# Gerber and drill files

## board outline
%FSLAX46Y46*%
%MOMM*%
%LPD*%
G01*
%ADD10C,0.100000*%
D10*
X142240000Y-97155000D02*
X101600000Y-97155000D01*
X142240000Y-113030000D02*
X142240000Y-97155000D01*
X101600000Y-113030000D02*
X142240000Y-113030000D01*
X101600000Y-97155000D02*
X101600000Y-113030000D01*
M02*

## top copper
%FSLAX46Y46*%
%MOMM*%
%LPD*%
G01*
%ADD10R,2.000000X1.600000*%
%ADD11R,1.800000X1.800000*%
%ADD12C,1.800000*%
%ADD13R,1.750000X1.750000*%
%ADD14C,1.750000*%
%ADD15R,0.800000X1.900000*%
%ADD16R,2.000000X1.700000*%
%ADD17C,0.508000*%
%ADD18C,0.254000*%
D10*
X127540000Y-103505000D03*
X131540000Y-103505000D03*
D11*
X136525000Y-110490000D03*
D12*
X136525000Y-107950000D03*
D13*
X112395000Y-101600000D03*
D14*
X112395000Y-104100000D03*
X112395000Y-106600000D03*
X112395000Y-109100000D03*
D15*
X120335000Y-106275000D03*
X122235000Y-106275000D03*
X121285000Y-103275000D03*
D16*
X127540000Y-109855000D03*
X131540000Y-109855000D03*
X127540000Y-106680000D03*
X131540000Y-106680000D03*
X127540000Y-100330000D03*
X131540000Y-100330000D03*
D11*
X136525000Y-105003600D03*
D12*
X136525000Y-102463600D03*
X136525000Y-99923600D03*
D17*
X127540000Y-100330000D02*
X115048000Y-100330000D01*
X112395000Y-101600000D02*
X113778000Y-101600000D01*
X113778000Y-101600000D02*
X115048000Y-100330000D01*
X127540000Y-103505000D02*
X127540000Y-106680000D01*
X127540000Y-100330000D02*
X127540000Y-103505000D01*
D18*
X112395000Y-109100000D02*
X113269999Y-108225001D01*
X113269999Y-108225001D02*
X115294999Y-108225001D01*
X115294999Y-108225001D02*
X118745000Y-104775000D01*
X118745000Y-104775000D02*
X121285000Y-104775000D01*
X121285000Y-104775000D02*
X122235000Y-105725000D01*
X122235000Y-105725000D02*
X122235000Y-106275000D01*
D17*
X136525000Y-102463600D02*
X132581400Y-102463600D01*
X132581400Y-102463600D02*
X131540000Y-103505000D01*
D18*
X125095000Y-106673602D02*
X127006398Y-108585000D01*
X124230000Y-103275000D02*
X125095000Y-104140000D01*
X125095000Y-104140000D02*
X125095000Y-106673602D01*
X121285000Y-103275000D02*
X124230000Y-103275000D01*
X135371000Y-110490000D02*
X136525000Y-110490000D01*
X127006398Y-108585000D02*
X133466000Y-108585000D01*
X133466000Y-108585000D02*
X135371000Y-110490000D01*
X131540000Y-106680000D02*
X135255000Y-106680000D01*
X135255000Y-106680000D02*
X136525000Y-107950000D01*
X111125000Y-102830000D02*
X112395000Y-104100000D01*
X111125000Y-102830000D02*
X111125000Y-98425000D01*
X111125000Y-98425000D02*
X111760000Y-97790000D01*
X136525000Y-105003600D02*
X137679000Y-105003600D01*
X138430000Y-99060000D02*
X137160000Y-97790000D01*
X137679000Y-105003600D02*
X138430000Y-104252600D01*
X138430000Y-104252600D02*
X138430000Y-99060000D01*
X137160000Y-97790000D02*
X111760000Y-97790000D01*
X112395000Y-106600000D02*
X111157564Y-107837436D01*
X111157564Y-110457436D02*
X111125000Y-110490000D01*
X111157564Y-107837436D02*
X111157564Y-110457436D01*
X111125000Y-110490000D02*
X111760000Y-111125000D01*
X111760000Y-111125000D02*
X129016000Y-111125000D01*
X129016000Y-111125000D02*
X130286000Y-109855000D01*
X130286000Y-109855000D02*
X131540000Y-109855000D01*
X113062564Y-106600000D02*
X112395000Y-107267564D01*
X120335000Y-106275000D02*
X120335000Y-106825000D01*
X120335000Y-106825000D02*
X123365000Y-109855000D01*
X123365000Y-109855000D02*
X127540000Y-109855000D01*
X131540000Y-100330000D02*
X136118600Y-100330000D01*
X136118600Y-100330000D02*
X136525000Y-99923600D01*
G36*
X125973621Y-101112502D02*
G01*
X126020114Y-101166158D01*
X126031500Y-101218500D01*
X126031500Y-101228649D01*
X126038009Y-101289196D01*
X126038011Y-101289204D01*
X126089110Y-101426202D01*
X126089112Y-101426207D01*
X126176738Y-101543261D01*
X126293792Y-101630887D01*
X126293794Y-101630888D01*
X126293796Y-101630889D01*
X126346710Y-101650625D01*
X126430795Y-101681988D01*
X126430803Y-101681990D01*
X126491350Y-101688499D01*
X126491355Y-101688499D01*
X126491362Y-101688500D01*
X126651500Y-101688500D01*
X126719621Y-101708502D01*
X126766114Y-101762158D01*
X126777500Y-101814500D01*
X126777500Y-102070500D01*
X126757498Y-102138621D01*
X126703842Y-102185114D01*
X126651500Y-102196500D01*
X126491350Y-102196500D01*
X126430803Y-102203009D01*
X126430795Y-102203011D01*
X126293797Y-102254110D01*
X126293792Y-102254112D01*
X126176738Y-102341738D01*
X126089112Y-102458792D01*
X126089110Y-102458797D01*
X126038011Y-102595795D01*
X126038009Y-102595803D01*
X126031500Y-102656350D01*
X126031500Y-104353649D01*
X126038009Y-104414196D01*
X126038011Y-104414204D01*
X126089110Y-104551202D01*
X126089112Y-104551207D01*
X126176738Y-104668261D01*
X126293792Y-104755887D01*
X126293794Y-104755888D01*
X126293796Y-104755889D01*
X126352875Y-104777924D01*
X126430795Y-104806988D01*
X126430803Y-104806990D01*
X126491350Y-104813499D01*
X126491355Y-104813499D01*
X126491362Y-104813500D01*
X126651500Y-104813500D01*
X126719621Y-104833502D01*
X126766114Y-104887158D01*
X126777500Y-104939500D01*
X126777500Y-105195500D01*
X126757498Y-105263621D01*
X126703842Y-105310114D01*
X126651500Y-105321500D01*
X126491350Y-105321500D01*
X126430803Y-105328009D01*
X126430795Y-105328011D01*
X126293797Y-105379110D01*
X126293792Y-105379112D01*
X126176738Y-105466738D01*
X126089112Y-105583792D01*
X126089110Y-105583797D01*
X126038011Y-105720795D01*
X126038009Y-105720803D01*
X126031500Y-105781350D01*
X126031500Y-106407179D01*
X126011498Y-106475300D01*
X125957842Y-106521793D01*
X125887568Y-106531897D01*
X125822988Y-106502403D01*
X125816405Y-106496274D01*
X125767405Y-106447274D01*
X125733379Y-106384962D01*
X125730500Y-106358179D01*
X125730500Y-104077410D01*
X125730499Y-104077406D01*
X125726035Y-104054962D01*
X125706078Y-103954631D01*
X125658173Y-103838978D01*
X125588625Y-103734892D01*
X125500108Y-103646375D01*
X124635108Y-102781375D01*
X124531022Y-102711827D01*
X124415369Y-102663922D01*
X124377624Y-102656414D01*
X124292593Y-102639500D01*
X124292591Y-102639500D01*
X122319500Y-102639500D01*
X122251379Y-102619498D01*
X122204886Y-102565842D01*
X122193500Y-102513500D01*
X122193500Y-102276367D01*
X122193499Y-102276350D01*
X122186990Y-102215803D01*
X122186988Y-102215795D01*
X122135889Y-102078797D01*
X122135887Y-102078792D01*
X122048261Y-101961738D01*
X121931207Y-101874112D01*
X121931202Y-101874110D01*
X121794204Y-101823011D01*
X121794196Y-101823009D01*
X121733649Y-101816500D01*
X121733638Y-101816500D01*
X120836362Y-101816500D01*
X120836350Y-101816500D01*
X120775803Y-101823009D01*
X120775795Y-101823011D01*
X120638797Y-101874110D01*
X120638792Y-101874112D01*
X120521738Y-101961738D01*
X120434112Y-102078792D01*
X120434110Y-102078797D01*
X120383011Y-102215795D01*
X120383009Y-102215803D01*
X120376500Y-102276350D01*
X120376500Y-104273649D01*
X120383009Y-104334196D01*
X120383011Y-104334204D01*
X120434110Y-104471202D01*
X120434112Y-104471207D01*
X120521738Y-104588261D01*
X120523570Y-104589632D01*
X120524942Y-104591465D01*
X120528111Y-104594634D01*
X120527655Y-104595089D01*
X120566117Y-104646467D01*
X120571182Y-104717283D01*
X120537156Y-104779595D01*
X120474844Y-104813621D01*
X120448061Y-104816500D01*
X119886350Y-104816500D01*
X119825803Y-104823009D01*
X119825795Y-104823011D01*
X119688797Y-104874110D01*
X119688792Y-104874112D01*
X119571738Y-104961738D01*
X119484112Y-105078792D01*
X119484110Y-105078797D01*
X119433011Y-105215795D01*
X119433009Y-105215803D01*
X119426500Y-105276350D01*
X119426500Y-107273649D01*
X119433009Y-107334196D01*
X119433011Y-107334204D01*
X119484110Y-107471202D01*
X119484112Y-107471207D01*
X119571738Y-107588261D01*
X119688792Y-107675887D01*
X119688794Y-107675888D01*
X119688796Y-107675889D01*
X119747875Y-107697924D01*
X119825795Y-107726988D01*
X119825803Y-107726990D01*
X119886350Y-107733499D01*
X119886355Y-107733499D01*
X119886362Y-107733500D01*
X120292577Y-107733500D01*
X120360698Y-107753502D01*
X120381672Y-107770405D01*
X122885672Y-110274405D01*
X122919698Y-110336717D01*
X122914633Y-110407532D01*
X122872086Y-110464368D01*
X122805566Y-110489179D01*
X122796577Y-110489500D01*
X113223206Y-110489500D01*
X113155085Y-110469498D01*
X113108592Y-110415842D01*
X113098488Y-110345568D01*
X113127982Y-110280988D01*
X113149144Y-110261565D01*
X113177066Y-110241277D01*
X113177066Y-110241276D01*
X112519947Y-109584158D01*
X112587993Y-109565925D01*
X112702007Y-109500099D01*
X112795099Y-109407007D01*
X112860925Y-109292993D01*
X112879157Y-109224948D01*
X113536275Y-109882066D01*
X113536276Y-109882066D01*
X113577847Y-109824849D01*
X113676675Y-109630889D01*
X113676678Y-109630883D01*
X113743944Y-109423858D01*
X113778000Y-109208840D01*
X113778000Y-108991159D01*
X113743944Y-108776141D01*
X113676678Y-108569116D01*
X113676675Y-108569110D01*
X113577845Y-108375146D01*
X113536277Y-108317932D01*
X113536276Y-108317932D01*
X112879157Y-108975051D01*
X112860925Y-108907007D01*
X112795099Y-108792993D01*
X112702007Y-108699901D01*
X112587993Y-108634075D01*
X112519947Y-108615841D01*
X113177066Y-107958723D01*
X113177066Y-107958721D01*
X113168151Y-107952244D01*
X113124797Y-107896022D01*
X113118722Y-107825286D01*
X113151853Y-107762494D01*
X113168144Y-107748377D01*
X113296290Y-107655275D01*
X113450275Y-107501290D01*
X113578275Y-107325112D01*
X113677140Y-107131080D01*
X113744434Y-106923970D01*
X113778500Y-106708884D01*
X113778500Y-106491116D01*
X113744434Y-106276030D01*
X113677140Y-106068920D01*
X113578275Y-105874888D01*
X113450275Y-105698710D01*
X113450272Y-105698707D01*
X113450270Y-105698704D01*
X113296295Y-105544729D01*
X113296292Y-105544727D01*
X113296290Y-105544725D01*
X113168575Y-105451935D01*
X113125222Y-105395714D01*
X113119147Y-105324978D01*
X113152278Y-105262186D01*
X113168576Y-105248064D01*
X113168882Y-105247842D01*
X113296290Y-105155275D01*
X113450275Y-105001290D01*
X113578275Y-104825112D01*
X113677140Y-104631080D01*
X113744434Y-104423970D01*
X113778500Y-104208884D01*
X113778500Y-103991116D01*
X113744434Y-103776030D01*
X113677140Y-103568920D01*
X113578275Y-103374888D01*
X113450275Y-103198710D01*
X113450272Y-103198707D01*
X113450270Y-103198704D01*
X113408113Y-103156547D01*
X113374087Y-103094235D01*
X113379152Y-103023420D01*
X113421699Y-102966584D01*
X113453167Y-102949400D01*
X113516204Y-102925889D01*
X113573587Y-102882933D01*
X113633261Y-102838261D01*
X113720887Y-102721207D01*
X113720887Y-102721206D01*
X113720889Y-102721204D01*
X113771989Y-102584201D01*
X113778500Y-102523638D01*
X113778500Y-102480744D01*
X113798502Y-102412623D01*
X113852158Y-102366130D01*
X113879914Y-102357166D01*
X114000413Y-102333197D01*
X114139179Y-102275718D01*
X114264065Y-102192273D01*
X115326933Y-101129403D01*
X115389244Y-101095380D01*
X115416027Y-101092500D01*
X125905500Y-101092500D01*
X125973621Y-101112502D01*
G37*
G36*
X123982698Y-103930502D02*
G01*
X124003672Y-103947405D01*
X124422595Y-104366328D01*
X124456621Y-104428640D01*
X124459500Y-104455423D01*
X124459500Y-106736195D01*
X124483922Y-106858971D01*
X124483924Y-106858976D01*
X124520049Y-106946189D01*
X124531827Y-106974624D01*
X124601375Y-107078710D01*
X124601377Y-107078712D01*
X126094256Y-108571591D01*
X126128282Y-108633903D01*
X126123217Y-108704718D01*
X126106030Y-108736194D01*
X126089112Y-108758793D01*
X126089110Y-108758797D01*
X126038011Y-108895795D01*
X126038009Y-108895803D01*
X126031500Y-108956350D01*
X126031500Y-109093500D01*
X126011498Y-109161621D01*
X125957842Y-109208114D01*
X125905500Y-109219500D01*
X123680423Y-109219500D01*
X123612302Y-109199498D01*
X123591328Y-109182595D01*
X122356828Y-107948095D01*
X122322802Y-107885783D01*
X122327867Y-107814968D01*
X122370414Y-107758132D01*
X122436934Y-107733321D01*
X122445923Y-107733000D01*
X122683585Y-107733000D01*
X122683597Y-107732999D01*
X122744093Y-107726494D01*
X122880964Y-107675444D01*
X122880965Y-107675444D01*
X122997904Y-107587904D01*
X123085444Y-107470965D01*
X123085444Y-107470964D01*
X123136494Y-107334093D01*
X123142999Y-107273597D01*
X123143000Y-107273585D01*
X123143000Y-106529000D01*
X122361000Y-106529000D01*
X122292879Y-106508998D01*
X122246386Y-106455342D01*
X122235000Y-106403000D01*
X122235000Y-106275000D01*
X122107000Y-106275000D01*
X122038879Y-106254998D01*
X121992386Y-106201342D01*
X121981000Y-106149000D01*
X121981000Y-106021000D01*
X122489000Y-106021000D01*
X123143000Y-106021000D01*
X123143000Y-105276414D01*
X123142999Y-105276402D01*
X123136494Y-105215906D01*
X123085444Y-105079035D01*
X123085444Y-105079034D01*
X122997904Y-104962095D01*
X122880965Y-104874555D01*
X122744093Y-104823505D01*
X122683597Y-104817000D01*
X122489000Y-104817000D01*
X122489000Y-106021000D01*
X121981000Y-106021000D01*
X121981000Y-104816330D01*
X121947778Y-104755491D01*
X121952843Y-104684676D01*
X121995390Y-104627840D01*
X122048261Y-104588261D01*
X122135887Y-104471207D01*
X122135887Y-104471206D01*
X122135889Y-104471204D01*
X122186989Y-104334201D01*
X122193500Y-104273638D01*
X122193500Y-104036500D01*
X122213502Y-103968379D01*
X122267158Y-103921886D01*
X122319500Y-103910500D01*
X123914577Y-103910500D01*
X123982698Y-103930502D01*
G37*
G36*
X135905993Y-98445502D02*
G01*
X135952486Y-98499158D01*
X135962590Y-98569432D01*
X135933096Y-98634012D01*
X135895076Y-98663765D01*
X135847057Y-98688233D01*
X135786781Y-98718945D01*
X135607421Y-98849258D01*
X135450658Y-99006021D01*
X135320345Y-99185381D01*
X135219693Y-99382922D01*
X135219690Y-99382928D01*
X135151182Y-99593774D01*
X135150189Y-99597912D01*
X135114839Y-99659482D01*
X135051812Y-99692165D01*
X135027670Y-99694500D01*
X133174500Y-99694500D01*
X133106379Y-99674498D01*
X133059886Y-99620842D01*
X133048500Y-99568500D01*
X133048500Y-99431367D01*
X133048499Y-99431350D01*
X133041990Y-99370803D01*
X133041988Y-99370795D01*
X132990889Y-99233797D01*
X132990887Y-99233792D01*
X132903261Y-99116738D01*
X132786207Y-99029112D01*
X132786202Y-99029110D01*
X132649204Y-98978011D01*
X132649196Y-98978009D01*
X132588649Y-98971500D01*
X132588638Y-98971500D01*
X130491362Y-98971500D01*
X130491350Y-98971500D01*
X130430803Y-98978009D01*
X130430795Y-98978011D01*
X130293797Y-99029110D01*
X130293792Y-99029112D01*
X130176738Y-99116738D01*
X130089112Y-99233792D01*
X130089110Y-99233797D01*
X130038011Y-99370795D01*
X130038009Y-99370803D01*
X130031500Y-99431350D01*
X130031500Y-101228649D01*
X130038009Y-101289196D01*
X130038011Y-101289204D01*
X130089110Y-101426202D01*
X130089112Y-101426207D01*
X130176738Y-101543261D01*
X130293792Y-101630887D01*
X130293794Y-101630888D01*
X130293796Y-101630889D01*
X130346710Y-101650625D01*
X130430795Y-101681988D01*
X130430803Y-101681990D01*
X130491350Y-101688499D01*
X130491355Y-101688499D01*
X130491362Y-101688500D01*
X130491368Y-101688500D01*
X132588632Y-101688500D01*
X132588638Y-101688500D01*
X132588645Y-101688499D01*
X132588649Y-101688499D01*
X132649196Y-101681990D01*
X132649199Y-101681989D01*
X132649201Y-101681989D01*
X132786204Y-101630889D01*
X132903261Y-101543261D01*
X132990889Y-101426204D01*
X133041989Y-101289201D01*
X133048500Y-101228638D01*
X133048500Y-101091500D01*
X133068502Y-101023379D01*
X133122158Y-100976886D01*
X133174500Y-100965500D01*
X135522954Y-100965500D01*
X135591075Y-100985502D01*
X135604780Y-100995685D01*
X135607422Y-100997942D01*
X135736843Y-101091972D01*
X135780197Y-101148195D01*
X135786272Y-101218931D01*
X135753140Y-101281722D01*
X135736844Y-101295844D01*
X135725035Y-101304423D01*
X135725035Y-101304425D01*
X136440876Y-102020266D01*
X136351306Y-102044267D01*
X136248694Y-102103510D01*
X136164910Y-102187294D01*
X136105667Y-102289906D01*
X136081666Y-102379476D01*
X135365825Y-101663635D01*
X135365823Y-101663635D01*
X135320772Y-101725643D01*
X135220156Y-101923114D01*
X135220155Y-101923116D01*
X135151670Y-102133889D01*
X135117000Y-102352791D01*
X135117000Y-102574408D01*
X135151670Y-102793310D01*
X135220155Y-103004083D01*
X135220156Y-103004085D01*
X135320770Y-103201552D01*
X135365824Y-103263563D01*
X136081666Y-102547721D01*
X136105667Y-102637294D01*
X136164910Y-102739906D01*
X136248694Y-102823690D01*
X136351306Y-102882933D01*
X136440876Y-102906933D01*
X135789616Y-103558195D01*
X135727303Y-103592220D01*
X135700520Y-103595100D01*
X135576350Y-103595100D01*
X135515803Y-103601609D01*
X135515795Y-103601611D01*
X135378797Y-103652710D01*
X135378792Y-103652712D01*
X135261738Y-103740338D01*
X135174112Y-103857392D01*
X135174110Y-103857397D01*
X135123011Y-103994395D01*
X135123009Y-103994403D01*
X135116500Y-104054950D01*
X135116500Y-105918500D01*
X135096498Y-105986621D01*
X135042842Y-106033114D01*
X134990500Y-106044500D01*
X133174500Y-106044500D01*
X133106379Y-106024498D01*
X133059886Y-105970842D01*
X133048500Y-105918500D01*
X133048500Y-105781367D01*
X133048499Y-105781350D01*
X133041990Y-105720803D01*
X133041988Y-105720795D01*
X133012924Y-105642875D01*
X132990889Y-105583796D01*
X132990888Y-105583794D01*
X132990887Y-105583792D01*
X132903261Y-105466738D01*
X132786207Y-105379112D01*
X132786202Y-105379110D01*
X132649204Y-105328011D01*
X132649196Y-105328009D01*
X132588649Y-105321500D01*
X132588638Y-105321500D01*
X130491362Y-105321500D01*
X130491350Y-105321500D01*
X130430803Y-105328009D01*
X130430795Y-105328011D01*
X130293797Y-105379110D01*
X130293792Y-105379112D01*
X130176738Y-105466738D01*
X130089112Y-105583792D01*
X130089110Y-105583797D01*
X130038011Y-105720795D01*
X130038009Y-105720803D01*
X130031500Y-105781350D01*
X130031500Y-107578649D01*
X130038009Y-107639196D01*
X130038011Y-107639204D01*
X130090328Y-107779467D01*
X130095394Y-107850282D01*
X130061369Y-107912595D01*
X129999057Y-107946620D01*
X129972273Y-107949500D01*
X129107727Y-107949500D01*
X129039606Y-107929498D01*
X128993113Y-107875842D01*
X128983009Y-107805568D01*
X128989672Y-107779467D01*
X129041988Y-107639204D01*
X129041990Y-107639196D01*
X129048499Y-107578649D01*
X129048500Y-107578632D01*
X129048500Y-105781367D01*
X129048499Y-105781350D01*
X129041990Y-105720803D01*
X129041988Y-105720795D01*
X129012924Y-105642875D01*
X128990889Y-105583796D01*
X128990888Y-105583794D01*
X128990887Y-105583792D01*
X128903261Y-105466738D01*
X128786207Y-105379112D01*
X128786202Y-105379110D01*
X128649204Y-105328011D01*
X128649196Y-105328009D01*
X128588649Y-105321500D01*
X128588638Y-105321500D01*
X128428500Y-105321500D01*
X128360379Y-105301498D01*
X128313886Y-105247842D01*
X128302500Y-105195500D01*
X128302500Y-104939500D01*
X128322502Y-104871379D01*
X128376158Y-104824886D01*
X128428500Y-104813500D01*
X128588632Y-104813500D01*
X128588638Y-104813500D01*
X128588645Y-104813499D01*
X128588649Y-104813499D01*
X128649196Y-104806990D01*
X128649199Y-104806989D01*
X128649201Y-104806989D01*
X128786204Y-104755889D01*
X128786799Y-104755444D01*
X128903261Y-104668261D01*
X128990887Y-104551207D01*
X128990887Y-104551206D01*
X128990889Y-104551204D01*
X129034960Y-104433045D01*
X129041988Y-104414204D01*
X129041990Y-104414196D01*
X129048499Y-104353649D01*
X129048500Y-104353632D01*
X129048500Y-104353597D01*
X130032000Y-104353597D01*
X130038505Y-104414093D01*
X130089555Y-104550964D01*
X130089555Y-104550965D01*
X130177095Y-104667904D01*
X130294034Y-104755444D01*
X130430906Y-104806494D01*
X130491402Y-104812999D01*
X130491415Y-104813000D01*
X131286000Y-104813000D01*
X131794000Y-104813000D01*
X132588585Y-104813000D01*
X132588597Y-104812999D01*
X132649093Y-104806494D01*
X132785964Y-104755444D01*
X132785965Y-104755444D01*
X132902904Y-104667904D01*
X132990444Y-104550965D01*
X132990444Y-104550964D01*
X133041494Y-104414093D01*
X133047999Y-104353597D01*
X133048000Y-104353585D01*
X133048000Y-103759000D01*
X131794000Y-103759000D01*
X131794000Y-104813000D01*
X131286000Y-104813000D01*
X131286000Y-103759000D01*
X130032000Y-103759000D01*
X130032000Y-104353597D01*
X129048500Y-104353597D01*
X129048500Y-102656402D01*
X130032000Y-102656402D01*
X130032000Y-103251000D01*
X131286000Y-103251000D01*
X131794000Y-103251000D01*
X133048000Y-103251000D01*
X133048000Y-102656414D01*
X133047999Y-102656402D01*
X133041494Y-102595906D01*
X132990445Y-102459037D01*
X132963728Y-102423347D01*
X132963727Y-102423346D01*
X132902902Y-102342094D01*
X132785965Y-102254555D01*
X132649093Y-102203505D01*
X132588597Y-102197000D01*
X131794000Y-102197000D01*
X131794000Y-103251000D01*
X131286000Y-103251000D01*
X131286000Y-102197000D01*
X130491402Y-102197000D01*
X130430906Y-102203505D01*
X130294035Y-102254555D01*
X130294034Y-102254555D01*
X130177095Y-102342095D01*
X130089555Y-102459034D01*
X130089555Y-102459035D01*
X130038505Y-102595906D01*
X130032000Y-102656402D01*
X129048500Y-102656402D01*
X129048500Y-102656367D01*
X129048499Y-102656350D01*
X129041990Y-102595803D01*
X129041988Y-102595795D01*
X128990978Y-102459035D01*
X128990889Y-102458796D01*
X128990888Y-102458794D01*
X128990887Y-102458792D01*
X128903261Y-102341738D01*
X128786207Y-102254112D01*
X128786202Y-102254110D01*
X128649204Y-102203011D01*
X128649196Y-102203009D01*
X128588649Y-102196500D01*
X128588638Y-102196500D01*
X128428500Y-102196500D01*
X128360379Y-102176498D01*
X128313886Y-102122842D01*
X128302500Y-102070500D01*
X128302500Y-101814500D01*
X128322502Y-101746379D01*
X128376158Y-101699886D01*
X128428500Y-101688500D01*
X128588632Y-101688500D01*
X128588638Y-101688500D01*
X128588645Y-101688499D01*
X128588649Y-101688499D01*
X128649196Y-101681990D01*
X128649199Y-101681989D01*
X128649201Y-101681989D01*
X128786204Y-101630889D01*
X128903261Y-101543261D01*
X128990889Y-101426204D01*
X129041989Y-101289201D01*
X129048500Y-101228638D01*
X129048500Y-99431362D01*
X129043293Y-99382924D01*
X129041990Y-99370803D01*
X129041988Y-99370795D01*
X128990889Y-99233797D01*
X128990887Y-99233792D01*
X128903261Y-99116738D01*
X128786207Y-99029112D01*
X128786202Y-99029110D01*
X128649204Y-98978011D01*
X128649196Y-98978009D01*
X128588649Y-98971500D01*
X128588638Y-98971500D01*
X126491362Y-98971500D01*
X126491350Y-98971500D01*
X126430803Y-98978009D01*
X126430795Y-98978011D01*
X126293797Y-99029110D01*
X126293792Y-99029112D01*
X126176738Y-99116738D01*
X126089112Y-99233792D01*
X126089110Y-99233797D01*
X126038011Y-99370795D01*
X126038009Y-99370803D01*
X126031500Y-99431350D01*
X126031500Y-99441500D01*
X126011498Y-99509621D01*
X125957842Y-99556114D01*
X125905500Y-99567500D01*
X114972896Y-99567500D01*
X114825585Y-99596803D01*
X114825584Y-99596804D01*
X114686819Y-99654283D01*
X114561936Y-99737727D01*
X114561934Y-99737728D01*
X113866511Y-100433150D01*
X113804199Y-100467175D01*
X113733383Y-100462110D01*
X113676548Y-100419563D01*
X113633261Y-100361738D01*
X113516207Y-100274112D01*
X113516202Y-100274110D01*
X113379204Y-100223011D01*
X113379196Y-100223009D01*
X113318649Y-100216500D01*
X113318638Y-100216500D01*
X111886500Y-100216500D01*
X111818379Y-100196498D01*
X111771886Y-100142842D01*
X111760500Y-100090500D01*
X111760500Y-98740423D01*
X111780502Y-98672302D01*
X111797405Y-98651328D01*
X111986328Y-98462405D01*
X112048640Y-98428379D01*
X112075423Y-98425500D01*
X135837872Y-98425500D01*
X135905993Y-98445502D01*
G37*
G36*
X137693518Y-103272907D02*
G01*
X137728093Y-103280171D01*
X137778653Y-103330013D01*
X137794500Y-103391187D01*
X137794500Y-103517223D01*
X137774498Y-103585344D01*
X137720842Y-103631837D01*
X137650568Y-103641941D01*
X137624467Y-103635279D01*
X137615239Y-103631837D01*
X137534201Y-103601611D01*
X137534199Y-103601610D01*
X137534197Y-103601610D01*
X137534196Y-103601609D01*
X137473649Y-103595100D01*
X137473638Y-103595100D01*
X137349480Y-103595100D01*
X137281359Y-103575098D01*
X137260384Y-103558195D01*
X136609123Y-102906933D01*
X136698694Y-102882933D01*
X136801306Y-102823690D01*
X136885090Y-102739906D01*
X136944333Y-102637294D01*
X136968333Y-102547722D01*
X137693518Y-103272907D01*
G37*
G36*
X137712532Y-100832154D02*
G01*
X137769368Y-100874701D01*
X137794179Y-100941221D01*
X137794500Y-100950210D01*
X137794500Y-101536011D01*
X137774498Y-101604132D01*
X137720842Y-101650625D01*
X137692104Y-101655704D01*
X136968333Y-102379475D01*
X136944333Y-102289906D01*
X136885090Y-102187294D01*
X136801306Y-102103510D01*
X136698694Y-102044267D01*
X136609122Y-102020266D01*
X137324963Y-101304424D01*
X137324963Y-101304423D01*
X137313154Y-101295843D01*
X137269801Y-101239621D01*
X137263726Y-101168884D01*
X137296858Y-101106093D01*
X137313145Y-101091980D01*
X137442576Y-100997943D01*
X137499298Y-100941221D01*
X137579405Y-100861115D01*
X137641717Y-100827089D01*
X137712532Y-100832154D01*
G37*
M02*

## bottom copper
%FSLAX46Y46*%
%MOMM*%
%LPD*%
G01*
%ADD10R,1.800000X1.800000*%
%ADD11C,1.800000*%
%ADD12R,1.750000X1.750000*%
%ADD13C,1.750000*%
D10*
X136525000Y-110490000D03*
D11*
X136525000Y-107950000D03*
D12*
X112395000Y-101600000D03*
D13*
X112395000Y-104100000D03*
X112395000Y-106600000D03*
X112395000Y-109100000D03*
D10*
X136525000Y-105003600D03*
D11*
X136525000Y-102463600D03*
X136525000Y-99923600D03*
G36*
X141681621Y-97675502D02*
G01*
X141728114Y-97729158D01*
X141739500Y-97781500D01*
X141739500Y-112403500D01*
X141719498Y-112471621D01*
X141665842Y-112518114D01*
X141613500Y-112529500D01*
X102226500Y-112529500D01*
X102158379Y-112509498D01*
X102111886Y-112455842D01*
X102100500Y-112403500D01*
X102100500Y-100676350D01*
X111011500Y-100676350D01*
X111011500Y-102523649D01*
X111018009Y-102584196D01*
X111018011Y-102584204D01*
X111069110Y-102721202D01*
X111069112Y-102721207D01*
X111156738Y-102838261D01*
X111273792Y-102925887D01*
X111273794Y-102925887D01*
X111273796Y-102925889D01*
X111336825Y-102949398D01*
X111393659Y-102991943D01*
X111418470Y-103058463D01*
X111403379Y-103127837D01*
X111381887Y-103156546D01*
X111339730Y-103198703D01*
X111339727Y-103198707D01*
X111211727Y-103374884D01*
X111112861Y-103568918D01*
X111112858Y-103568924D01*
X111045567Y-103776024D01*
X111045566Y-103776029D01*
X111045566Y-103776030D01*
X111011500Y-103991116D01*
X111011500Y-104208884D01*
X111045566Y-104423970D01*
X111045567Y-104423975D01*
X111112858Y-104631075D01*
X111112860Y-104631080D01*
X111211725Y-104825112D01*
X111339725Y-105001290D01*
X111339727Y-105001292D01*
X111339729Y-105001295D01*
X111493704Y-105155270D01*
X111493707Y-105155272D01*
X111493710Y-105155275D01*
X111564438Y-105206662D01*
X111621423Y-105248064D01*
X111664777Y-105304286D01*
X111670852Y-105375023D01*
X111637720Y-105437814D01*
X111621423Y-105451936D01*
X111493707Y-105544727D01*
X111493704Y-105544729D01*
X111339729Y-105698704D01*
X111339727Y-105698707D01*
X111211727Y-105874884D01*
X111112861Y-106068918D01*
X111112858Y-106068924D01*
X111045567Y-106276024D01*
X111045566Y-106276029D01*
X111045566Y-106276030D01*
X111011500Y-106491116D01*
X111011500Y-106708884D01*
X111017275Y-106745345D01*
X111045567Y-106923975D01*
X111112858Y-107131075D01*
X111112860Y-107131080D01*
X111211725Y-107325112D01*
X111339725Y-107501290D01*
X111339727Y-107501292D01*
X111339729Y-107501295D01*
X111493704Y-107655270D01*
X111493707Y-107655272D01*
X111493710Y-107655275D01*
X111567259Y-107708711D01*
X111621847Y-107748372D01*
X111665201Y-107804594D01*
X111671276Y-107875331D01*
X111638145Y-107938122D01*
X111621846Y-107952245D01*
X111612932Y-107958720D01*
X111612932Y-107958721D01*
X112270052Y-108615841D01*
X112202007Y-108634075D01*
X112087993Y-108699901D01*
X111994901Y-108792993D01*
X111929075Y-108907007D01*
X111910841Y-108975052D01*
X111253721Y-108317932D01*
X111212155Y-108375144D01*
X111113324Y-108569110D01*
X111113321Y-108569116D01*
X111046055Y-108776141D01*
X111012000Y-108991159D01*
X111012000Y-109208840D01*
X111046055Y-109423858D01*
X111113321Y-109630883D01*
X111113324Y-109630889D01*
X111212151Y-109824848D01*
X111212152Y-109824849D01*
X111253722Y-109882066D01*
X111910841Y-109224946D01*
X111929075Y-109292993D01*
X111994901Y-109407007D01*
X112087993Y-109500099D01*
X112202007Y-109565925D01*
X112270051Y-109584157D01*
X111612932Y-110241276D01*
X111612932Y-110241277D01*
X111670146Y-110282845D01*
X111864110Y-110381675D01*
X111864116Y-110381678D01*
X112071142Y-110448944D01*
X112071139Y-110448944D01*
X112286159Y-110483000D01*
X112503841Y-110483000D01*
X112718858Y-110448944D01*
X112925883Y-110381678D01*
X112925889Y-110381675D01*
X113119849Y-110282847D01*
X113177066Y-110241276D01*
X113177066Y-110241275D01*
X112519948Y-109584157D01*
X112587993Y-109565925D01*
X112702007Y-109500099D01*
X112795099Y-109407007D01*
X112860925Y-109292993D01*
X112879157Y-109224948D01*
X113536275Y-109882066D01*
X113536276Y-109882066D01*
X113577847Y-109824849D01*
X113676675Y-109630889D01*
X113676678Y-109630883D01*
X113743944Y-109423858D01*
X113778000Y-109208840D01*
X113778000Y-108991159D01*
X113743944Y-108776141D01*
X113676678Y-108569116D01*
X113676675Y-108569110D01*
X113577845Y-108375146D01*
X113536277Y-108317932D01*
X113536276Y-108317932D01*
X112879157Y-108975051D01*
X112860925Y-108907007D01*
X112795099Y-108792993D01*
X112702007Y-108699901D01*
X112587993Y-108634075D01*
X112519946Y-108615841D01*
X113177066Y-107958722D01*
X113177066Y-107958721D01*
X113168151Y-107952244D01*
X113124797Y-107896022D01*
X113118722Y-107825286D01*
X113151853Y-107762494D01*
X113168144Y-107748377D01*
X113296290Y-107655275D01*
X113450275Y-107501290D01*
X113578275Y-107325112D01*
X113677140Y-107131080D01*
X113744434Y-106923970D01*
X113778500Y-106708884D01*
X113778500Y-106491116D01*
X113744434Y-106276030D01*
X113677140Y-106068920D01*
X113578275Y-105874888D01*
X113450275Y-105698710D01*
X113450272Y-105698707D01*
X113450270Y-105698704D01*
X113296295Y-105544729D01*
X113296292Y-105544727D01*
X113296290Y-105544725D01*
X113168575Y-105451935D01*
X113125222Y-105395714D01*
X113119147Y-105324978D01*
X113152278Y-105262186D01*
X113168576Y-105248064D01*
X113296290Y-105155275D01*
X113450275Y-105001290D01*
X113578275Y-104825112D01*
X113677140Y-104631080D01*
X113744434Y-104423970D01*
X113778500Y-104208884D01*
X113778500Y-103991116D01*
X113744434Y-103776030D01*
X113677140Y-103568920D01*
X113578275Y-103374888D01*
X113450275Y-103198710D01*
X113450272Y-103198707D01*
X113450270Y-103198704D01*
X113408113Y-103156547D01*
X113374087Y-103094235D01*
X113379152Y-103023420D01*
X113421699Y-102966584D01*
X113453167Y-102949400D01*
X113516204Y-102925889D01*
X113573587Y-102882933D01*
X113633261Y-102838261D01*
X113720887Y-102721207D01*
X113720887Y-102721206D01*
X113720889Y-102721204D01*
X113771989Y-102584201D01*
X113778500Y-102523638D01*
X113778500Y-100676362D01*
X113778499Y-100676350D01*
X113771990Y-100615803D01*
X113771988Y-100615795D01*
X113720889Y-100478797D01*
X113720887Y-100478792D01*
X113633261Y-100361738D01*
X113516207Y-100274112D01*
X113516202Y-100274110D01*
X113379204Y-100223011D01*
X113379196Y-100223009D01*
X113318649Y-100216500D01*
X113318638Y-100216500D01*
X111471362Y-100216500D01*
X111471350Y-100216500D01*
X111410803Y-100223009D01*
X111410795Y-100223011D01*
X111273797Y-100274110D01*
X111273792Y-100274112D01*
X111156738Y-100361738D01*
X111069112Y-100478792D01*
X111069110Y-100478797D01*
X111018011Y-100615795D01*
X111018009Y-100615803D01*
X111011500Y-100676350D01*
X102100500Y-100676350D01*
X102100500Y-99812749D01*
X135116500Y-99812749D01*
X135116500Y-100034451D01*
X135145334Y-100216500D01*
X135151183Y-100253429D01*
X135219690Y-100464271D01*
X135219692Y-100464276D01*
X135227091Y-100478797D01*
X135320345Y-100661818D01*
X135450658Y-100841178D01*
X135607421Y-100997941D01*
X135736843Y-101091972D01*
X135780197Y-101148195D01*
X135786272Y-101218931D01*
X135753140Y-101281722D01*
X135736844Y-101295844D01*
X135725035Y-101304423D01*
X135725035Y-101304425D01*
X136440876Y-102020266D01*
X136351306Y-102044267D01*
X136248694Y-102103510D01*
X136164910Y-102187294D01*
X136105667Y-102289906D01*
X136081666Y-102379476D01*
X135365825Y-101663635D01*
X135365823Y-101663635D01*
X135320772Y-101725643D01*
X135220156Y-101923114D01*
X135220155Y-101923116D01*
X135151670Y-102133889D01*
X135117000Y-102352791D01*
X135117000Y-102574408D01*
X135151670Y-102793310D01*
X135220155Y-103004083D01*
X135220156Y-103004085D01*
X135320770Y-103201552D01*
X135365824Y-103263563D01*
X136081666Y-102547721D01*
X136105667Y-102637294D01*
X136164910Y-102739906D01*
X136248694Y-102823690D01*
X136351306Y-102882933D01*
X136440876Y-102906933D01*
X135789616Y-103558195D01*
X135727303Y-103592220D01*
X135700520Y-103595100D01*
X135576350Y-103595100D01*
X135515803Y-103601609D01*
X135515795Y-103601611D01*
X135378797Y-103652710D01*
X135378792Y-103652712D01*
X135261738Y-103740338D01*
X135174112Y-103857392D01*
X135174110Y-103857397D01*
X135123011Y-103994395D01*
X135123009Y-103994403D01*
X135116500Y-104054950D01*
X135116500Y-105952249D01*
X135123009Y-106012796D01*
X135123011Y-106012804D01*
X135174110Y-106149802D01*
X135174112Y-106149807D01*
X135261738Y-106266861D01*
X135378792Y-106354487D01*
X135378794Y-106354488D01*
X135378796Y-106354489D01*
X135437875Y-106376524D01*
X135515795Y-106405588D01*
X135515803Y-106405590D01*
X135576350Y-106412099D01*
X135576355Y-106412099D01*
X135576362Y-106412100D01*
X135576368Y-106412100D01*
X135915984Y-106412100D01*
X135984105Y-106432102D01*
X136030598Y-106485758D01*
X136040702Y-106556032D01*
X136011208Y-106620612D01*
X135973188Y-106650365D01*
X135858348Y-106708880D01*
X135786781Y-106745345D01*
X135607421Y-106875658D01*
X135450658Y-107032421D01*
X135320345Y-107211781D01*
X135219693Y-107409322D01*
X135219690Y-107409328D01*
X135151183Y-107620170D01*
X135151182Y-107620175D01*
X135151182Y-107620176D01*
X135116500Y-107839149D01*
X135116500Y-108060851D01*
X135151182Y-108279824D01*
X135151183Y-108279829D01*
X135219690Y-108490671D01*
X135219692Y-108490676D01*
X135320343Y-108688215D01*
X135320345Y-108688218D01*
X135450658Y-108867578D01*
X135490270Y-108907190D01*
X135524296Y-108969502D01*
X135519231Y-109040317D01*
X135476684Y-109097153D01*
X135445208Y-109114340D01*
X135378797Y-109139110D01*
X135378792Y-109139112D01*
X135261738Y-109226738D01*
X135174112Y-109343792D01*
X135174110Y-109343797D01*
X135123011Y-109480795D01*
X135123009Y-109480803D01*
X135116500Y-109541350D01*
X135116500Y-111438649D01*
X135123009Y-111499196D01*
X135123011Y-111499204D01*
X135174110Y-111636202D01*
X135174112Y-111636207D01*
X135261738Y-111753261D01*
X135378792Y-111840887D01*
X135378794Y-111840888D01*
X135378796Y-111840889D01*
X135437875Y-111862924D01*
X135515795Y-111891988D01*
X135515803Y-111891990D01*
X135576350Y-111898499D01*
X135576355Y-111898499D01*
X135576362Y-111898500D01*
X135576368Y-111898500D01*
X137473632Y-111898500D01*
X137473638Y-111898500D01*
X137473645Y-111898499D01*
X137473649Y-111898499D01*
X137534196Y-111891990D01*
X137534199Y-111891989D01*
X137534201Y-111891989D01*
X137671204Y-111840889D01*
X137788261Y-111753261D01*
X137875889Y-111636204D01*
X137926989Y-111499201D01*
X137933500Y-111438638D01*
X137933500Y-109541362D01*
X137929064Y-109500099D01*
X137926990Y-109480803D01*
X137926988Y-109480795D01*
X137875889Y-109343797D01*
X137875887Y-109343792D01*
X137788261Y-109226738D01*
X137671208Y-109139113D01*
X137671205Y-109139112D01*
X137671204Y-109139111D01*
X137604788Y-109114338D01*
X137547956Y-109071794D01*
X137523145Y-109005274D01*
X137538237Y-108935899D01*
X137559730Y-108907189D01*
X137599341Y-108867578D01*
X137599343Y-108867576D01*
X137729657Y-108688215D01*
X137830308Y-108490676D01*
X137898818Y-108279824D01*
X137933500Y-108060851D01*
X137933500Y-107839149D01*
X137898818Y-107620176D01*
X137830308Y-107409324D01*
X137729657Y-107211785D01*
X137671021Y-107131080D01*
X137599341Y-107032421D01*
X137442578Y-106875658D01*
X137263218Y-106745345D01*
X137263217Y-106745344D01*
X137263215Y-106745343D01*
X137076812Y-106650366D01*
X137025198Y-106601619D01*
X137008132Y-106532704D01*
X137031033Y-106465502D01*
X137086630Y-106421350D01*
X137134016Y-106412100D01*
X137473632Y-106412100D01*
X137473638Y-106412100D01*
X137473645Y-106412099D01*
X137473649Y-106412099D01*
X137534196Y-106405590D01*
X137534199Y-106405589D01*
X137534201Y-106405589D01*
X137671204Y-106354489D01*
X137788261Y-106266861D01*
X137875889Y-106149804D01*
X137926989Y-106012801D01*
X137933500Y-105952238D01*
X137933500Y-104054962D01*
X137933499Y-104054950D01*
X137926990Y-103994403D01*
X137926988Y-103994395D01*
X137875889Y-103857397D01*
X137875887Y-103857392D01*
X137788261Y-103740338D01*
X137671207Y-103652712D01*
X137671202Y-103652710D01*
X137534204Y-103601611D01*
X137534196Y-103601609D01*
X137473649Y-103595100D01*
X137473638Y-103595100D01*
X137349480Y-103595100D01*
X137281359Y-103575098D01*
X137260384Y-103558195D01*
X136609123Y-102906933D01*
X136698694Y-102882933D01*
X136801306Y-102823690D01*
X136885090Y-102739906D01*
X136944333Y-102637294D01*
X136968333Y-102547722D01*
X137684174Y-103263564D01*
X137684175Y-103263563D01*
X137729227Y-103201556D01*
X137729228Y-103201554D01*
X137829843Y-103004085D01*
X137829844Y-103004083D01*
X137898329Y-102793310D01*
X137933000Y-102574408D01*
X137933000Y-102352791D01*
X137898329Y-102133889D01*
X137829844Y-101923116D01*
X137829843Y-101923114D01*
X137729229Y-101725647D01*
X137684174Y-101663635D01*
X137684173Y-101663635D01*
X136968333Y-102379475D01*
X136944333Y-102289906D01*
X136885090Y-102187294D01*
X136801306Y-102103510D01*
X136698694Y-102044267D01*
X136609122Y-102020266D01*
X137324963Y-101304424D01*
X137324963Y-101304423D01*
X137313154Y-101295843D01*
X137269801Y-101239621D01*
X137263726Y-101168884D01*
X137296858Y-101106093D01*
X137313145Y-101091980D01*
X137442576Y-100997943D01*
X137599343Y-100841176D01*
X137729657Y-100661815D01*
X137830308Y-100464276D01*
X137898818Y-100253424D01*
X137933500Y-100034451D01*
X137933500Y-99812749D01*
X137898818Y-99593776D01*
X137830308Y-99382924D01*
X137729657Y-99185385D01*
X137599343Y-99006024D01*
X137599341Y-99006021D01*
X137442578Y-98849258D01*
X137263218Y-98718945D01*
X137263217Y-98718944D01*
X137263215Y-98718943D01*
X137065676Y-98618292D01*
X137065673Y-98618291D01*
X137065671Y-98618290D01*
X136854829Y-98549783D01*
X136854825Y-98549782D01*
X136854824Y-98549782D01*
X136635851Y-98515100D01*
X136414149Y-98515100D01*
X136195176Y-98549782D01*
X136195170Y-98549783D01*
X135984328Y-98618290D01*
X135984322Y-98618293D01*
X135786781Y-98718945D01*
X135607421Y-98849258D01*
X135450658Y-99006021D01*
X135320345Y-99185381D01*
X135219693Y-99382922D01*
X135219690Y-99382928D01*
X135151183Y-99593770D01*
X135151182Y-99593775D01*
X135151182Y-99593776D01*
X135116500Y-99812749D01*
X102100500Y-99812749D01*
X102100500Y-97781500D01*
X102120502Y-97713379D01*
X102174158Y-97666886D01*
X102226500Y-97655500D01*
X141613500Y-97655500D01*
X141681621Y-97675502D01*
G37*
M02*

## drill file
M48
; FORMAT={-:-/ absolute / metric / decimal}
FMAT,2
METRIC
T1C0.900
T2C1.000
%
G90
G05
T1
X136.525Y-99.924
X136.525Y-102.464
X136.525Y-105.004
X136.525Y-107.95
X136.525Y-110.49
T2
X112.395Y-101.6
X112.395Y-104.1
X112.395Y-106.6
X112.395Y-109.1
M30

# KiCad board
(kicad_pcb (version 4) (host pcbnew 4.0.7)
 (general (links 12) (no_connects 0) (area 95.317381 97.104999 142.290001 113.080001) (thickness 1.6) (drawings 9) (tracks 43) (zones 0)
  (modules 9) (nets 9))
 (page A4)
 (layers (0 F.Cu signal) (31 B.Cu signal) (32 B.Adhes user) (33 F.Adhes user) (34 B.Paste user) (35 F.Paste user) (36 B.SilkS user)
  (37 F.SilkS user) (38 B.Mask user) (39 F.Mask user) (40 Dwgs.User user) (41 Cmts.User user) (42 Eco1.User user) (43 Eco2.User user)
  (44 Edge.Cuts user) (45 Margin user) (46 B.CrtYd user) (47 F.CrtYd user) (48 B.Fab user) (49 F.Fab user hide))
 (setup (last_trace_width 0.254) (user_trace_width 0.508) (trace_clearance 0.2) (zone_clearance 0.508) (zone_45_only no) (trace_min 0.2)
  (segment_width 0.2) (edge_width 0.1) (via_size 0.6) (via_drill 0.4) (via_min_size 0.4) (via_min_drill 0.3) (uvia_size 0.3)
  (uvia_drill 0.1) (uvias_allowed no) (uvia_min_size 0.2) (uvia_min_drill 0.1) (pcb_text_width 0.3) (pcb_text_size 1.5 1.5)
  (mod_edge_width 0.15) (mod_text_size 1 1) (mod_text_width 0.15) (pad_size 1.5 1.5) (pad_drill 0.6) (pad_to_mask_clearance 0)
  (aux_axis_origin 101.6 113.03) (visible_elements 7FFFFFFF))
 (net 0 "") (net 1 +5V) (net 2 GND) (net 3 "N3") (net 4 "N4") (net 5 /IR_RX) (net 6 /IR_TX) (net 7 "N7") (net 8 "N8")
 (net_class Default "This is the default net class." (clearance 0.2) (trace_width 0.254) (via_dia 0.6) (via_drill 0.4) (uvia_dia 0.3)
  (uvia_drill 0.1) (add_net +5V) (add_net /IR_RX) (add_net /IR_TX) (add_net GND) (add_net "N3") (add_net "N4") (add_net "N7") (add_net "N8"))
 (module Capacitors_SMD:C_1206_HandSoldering (layer F.Cu) (at 129.54 103.505)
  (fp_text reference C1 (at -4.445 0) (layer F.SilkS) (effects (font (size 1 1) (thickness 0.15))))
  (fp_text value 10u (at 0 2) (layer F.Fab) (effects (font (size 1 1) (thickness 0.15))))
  (pad 1 smd rect (at -2 0) (size 2 1.6) (layers F.Cu F.Paste F.Mask) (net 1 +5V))
  (pad 2 smd rect (at 2 0) (size 2 1.6) (layers F.Cu F.Paste F.Mask) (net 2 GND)))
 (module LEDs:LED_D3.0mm (layer F.Cu) (at 136.525 110.49 90)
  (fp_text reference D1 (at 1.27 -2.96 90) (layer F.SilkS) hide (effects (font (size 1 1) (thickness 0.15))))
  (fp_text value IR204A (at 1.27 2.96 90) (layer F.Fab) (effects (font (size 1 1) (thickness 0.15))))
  (pad 1 thru_hole rect (at 0 0 90) (size 1.8 1.8) (drill 0.9) (layers *.Cu *.Mask) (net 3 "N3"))
  (pad 2 thru_hole circle (at 2.54 0 90) (size 1.8 1.8) (drill 0.9) (layers *.Cu *.Mask) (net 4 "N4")))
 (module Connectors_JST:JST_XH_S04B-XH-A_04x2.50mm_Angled (layer F.Cu) (at 112.395 101.6 270)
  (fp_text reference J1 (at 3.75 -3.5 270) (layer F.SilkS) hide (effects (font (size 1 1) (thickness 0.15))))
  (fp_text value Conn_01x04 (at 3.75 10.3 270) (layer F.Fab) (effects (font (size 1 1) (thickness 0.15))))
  (pad 1 thru_hole rect (at 0 0 270) (size 1.75 1.75) (drill 1) (layers *.Cu *.Mask F.SilkS) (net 1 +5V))
  (pad 2 thru_hole circle (at 2.5 0 270) (size 1.75 1.75) (drill 1) (layers *.Cu *.Mask F.SilkS) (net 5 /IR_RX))
  (pad 3 thru_hole circle (at 5 0 270) (size 1.75 1.75) (drill 1) (layers *.Cu *.Mask F.SilkS) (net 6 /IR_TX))
  (pad 4 thru_hole circle (at 7.5 0 270) (size 1.75 1.75) (drill 1) (layers *.Cu *.Mask F.SilkS) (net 2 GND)))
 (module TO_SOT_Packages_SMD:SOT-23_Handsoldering (layer F.Cu) (at 121.285 104.775 90)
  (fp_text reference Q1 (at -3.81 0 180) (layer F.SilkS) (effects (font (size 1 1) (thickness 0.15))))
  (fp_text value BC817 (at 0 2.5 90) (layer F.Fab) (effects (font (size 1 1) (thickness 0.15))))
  (pad 1 smd rect (at -1.5 -0.95 90) (size 1.9 0.8) (layers F.Cu F.Paste F.Mask) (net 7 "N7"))
  (pad 2 smd rect (at -1.5 0.95 90) (size 1.9 0.8) (layers F.Cu F.Paste F.Mask) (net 2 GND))
  (pad 3 smd rect (at 1.5 0 90) (size 1.9 0.8) (layers F.Cu F.Paste F.Mask) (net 3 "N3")))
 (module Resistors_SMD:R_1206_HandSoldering (layer F.Cu) (at 129.54 109.855)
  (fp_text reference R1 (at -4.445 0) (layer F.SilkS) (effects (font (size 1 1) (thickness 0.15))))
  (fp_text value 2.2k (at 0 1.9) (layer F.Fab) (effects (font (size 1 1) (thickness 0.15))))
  (pad 1 smd rect (at -2 0) (size 2 1.7) (layers F.Cu F.Paste F.Mask) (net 7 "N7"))
  (pad 2 smd rect (at 2 0) (size 2 1.7) (layers F.Cu F.Paste F.Mask) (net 6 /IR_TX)))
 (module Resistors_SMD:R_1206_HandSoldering (layer F.Cu) (at 129.54 106.68)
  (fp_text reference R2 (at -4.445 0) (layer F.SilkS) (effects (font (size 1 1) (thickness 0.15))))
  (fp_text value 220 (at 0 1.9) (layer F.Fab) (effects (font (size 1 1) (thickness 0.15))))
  (pad 1 smd rect (at -2 0) (size 2 1.7) (layers F.Cu F.Paste F.Mask) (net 1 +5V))
  (pad 2 smd rect (at 2 0) (size 2 1.7) (layers F.Cu F.Paste F.Mask) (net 4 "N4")))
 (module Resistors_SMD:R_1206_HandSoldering (layer F.Cu) (at 129.54 100.33)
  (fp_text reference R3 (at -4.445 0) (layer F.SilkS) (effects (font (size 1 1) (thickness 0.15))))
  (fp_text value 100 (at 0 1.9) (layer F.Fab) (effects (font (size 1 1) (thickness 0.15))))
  (pad 1 smd rect (at -2 0) (size 2 1.7) (layers F.Cu F.Paste F.Mask) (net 1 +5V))
  (pad 2 smd rect (at 2 0) (size 2 1.7) (layers F.Cu F.Paste F.Mask) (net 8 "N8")))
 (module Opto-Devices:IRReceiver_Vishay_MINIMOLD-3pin (layer F.Cu) (at 136.525 105.0036 90)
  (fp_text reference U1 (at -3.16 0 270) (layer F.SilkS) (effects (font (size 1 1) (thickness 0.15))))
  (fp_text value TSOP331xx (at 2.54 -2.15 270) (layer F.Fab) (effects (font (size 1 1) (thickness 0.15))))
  (pad 1 thru_hole rect (at 0 0 90) (size 1.8 1.8) (drill 0.9) (layers *.Cu *.Mask) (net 5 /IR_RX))
  (pad 2 thru_hole circle (at 2.54 0 90) (size 1.8 1.8) (drill 0.9) (layers *.Cu *.Mask) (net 2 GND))
  (pad 3 thru_hole circle (at 5.08 0 90) (size 1.8 1.8) (drill 0.9) (layers *.Cu *.Mask) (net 8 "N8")))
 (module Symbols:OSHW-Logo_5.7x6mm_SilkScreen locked (layer B.Cu) (at 107.315 105.41)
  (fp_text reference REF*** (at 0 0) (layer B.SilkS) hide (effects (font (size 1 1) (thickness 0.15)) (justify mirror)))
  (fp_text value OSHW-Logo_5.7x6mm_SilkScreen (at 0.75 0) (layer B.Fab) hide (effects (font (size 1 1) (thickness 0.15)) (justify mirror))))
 (gr_line (start 142.24 97.155) (end 101.6 97.155) (layer Edge.Cuts) (width 0.1))
 (gr_line (start 142.24 113.03) (end 142.24 97.155) (layer Edge.Cuts) (width 0.1))
 (gr_line (start 101.6 113.03) (end 142.24 113.03) (layer Edge.Cuts) (width 0.1))
 (gr_line (start 101.6 97.155) (end 101.6 113.03) (layer Edge.Cuts) (width 0.1))
 (segment (start 127.54 100.33) (end 115.048 100.33) (width 0.508) (layer F.Cu) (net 1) (status 10))
 (segment (start 112.395 101.6) (end 113.778 101.6) (width 0.508) (layer F.Cu) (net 1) (status 10))
 (segment (start 113.778 101.6) (end 115.048 100.33) (width 0.508) (layer F.Cu) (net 1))
 (segment (start 127.54 103.505) (end 127.54 106.68) (width 0.508) (layer F.Cu) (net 1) (status 30))
 (segment (start 127.54 100.33) (end 127.54 103.505) (width 0.508) (layer F.Cu) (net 1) (status 30))
 (segment (start 112.395 109.1) (end 113.269999 108.225001) (width 0.254) (layer F.Cu) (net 2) (status 10))
 (segment (start 113.269999 108.225001) (end 115.294999 108.225001) (width 0.254) (layer F.Cu) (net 2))
 (segment (start 115.294999 108.225001) (end 118.745 104.775) (width 0.254) (layer F.Cu) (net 2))
 (segment (start 118.745 104.775) (end 121.285 104.775) (width 0.254) (layer F.Cu) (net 2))
 (segment (start 121.285 104.775) (end 122.235 105.725) (width 0.254) (layer F.Cu) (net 2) (status 20))
 (segment (start 122.235 105.725) (end 122.235 106.275) (width 0.254) (layer F.Cu) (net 2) (status 30))
 (segment (start 136.525 102.4636) (end 132.5814 102.4636) (width 0.508) (layer F.Cu) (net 2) (status 10))
 (segment (start 132.5814 102.4636) (end 131.54 103.505) (width 0.508) (layer F.Cu) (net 2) (status 20))
 (segment (start 125.095 106.673602) (end 127.006398 108.585) (width 0.254) (layer F.Cu) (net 3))
 (segment (start 124.23 103.275) (end 125.095 104.14) (width 0.254) (layer F.Cu) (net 3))
 (segment (start 125.095 104.14) (end 125.095 106.673602) (width 0.254) (layer F.Cu) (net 3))
 (segment (start 121.285 103.275) (end 124.23 103.275) (width 0.254) (layer F.Cu) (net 3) (status 10))
 (segment (start 135.371 110.49) (end 136.525 110.49) (width 0.254) (layer F.Cu) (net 3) (status 20))
 (segment (start 127.006398 108.585) (end 133.466 108.585) (width 0.254) (layer F.Cu) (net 3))
 (segment (start 133.466 108.585) (end 135.371 110.49) (width 0.254) (layer F.Cu) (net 3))
 (segment (start 131.54 106.68) (end 135.255 106.68) (width 0.254) (layer F.Cu) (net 4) (status 10))
 (segment (start 135.255 106.68) (end 136.525 107.95) (width 0.254) (layer F.Cu) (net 4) (status 20))
 (segment (start 111.125 102.83) (end 112.395 104.1) (width 0.254) (layer F.Cu) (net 5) (status 20))
 (segment (start 111.125 102.83) (end 111.125 98.425) (width 0.254) (layer F.Cu) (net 5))
 (segment (start 111.125 98.425) (end 111.76 97.79) (width 0.254) (layer F.Cu) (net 5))
 (segment (start 136.525 105.0036) (end 137.679 105.0036) (width 0.254) (layer F.Cu) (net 5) (status 10))
 (segment (start 138.43 99.06) (end 137.16 97.79) (width 0.254) (layer F.Cu) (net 5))
 (segment (start 137.679 105.0036) (end 138.43 104.2526) (width 0.254) (layer F.Cu) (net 5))
 (segment (start 138.43 104.2526) (end 138.43 99.06) (width 0.254) (layer F.Cu) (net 5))
 (segment (start 137.16 97.79) (end 111.76 97.79) (width 0.254) (layer F.Cu) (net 5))
 (segment (start 112.395 106.6) (end 111.157564 107.837436) (width 0.254) (layer F.Cu) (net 6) (status 10))
 (segment (start 111.157564 110.457436) (end 111.125 110.49) (width 0.254) (layer F.Cu) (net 6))
 (segment (start 111.157564 107.837436) (end 111.157564 110.457436) (width 0.254) (layer F.Cu) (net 6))
 (segment (start 111.125 110.49) (end 111.76 111.125) (width 0.254) (layer F.Cu) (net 6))
 (segment (start 111.76 111.125) (end 129.016 111.125) (width 0.254) (layer F.Cu) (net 6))
 (segment (start 129.016 111.125) (end 130.286 109.855) (width 0.254) (layer F.Cu) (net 6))
 (segment (start 130.286 109.855) (end 131.54 109.855) (width 0.254) (layer F.Cu) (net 6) (status 20))
 (segment (start 113.062564 106.6) (end 112.395 107.267564) (width 0.254) (layer F.Cu) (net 6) (status 30))
 (segment (start 120.335 106.275) (end 120.335 106.825) (width 0.254) (layer F.Cu) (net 7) (status 30))
 (segment (start 120.335 106.825) (end 123.365 109.855) (width 0.254) (layer F.Cu) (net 7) (status 10))
 (segment (start 123.365 109.855) (end 127.54 109.855) (width 0.254) (layer F.Cu) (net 7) (status 20))
 (segment (start 131.54 100.33) (end 136.1186 100.33) (width 0.254) (layer F.Cu) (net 8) (status 30))
 (segment (start 136.1186 100.33) (end 136.525 99.9236) (width 0.254) (layer F.Cu) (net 8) (status 30))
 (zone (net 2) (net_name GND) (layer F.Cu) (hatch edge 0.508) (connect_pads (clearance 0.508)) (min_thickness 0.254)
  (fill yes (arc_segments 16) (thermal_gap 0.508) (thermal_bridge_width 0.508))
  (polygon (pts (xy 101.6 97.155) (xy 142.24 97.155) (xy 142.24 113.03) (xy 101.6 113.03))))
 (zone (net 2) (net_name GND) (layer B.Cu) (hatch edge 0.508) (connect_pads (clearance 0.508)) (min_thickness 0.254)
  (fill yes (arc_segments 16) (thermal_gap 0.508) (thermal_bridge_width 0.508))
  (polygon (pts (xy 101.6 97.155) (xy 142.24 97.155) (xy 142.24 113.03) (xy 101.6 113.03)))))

